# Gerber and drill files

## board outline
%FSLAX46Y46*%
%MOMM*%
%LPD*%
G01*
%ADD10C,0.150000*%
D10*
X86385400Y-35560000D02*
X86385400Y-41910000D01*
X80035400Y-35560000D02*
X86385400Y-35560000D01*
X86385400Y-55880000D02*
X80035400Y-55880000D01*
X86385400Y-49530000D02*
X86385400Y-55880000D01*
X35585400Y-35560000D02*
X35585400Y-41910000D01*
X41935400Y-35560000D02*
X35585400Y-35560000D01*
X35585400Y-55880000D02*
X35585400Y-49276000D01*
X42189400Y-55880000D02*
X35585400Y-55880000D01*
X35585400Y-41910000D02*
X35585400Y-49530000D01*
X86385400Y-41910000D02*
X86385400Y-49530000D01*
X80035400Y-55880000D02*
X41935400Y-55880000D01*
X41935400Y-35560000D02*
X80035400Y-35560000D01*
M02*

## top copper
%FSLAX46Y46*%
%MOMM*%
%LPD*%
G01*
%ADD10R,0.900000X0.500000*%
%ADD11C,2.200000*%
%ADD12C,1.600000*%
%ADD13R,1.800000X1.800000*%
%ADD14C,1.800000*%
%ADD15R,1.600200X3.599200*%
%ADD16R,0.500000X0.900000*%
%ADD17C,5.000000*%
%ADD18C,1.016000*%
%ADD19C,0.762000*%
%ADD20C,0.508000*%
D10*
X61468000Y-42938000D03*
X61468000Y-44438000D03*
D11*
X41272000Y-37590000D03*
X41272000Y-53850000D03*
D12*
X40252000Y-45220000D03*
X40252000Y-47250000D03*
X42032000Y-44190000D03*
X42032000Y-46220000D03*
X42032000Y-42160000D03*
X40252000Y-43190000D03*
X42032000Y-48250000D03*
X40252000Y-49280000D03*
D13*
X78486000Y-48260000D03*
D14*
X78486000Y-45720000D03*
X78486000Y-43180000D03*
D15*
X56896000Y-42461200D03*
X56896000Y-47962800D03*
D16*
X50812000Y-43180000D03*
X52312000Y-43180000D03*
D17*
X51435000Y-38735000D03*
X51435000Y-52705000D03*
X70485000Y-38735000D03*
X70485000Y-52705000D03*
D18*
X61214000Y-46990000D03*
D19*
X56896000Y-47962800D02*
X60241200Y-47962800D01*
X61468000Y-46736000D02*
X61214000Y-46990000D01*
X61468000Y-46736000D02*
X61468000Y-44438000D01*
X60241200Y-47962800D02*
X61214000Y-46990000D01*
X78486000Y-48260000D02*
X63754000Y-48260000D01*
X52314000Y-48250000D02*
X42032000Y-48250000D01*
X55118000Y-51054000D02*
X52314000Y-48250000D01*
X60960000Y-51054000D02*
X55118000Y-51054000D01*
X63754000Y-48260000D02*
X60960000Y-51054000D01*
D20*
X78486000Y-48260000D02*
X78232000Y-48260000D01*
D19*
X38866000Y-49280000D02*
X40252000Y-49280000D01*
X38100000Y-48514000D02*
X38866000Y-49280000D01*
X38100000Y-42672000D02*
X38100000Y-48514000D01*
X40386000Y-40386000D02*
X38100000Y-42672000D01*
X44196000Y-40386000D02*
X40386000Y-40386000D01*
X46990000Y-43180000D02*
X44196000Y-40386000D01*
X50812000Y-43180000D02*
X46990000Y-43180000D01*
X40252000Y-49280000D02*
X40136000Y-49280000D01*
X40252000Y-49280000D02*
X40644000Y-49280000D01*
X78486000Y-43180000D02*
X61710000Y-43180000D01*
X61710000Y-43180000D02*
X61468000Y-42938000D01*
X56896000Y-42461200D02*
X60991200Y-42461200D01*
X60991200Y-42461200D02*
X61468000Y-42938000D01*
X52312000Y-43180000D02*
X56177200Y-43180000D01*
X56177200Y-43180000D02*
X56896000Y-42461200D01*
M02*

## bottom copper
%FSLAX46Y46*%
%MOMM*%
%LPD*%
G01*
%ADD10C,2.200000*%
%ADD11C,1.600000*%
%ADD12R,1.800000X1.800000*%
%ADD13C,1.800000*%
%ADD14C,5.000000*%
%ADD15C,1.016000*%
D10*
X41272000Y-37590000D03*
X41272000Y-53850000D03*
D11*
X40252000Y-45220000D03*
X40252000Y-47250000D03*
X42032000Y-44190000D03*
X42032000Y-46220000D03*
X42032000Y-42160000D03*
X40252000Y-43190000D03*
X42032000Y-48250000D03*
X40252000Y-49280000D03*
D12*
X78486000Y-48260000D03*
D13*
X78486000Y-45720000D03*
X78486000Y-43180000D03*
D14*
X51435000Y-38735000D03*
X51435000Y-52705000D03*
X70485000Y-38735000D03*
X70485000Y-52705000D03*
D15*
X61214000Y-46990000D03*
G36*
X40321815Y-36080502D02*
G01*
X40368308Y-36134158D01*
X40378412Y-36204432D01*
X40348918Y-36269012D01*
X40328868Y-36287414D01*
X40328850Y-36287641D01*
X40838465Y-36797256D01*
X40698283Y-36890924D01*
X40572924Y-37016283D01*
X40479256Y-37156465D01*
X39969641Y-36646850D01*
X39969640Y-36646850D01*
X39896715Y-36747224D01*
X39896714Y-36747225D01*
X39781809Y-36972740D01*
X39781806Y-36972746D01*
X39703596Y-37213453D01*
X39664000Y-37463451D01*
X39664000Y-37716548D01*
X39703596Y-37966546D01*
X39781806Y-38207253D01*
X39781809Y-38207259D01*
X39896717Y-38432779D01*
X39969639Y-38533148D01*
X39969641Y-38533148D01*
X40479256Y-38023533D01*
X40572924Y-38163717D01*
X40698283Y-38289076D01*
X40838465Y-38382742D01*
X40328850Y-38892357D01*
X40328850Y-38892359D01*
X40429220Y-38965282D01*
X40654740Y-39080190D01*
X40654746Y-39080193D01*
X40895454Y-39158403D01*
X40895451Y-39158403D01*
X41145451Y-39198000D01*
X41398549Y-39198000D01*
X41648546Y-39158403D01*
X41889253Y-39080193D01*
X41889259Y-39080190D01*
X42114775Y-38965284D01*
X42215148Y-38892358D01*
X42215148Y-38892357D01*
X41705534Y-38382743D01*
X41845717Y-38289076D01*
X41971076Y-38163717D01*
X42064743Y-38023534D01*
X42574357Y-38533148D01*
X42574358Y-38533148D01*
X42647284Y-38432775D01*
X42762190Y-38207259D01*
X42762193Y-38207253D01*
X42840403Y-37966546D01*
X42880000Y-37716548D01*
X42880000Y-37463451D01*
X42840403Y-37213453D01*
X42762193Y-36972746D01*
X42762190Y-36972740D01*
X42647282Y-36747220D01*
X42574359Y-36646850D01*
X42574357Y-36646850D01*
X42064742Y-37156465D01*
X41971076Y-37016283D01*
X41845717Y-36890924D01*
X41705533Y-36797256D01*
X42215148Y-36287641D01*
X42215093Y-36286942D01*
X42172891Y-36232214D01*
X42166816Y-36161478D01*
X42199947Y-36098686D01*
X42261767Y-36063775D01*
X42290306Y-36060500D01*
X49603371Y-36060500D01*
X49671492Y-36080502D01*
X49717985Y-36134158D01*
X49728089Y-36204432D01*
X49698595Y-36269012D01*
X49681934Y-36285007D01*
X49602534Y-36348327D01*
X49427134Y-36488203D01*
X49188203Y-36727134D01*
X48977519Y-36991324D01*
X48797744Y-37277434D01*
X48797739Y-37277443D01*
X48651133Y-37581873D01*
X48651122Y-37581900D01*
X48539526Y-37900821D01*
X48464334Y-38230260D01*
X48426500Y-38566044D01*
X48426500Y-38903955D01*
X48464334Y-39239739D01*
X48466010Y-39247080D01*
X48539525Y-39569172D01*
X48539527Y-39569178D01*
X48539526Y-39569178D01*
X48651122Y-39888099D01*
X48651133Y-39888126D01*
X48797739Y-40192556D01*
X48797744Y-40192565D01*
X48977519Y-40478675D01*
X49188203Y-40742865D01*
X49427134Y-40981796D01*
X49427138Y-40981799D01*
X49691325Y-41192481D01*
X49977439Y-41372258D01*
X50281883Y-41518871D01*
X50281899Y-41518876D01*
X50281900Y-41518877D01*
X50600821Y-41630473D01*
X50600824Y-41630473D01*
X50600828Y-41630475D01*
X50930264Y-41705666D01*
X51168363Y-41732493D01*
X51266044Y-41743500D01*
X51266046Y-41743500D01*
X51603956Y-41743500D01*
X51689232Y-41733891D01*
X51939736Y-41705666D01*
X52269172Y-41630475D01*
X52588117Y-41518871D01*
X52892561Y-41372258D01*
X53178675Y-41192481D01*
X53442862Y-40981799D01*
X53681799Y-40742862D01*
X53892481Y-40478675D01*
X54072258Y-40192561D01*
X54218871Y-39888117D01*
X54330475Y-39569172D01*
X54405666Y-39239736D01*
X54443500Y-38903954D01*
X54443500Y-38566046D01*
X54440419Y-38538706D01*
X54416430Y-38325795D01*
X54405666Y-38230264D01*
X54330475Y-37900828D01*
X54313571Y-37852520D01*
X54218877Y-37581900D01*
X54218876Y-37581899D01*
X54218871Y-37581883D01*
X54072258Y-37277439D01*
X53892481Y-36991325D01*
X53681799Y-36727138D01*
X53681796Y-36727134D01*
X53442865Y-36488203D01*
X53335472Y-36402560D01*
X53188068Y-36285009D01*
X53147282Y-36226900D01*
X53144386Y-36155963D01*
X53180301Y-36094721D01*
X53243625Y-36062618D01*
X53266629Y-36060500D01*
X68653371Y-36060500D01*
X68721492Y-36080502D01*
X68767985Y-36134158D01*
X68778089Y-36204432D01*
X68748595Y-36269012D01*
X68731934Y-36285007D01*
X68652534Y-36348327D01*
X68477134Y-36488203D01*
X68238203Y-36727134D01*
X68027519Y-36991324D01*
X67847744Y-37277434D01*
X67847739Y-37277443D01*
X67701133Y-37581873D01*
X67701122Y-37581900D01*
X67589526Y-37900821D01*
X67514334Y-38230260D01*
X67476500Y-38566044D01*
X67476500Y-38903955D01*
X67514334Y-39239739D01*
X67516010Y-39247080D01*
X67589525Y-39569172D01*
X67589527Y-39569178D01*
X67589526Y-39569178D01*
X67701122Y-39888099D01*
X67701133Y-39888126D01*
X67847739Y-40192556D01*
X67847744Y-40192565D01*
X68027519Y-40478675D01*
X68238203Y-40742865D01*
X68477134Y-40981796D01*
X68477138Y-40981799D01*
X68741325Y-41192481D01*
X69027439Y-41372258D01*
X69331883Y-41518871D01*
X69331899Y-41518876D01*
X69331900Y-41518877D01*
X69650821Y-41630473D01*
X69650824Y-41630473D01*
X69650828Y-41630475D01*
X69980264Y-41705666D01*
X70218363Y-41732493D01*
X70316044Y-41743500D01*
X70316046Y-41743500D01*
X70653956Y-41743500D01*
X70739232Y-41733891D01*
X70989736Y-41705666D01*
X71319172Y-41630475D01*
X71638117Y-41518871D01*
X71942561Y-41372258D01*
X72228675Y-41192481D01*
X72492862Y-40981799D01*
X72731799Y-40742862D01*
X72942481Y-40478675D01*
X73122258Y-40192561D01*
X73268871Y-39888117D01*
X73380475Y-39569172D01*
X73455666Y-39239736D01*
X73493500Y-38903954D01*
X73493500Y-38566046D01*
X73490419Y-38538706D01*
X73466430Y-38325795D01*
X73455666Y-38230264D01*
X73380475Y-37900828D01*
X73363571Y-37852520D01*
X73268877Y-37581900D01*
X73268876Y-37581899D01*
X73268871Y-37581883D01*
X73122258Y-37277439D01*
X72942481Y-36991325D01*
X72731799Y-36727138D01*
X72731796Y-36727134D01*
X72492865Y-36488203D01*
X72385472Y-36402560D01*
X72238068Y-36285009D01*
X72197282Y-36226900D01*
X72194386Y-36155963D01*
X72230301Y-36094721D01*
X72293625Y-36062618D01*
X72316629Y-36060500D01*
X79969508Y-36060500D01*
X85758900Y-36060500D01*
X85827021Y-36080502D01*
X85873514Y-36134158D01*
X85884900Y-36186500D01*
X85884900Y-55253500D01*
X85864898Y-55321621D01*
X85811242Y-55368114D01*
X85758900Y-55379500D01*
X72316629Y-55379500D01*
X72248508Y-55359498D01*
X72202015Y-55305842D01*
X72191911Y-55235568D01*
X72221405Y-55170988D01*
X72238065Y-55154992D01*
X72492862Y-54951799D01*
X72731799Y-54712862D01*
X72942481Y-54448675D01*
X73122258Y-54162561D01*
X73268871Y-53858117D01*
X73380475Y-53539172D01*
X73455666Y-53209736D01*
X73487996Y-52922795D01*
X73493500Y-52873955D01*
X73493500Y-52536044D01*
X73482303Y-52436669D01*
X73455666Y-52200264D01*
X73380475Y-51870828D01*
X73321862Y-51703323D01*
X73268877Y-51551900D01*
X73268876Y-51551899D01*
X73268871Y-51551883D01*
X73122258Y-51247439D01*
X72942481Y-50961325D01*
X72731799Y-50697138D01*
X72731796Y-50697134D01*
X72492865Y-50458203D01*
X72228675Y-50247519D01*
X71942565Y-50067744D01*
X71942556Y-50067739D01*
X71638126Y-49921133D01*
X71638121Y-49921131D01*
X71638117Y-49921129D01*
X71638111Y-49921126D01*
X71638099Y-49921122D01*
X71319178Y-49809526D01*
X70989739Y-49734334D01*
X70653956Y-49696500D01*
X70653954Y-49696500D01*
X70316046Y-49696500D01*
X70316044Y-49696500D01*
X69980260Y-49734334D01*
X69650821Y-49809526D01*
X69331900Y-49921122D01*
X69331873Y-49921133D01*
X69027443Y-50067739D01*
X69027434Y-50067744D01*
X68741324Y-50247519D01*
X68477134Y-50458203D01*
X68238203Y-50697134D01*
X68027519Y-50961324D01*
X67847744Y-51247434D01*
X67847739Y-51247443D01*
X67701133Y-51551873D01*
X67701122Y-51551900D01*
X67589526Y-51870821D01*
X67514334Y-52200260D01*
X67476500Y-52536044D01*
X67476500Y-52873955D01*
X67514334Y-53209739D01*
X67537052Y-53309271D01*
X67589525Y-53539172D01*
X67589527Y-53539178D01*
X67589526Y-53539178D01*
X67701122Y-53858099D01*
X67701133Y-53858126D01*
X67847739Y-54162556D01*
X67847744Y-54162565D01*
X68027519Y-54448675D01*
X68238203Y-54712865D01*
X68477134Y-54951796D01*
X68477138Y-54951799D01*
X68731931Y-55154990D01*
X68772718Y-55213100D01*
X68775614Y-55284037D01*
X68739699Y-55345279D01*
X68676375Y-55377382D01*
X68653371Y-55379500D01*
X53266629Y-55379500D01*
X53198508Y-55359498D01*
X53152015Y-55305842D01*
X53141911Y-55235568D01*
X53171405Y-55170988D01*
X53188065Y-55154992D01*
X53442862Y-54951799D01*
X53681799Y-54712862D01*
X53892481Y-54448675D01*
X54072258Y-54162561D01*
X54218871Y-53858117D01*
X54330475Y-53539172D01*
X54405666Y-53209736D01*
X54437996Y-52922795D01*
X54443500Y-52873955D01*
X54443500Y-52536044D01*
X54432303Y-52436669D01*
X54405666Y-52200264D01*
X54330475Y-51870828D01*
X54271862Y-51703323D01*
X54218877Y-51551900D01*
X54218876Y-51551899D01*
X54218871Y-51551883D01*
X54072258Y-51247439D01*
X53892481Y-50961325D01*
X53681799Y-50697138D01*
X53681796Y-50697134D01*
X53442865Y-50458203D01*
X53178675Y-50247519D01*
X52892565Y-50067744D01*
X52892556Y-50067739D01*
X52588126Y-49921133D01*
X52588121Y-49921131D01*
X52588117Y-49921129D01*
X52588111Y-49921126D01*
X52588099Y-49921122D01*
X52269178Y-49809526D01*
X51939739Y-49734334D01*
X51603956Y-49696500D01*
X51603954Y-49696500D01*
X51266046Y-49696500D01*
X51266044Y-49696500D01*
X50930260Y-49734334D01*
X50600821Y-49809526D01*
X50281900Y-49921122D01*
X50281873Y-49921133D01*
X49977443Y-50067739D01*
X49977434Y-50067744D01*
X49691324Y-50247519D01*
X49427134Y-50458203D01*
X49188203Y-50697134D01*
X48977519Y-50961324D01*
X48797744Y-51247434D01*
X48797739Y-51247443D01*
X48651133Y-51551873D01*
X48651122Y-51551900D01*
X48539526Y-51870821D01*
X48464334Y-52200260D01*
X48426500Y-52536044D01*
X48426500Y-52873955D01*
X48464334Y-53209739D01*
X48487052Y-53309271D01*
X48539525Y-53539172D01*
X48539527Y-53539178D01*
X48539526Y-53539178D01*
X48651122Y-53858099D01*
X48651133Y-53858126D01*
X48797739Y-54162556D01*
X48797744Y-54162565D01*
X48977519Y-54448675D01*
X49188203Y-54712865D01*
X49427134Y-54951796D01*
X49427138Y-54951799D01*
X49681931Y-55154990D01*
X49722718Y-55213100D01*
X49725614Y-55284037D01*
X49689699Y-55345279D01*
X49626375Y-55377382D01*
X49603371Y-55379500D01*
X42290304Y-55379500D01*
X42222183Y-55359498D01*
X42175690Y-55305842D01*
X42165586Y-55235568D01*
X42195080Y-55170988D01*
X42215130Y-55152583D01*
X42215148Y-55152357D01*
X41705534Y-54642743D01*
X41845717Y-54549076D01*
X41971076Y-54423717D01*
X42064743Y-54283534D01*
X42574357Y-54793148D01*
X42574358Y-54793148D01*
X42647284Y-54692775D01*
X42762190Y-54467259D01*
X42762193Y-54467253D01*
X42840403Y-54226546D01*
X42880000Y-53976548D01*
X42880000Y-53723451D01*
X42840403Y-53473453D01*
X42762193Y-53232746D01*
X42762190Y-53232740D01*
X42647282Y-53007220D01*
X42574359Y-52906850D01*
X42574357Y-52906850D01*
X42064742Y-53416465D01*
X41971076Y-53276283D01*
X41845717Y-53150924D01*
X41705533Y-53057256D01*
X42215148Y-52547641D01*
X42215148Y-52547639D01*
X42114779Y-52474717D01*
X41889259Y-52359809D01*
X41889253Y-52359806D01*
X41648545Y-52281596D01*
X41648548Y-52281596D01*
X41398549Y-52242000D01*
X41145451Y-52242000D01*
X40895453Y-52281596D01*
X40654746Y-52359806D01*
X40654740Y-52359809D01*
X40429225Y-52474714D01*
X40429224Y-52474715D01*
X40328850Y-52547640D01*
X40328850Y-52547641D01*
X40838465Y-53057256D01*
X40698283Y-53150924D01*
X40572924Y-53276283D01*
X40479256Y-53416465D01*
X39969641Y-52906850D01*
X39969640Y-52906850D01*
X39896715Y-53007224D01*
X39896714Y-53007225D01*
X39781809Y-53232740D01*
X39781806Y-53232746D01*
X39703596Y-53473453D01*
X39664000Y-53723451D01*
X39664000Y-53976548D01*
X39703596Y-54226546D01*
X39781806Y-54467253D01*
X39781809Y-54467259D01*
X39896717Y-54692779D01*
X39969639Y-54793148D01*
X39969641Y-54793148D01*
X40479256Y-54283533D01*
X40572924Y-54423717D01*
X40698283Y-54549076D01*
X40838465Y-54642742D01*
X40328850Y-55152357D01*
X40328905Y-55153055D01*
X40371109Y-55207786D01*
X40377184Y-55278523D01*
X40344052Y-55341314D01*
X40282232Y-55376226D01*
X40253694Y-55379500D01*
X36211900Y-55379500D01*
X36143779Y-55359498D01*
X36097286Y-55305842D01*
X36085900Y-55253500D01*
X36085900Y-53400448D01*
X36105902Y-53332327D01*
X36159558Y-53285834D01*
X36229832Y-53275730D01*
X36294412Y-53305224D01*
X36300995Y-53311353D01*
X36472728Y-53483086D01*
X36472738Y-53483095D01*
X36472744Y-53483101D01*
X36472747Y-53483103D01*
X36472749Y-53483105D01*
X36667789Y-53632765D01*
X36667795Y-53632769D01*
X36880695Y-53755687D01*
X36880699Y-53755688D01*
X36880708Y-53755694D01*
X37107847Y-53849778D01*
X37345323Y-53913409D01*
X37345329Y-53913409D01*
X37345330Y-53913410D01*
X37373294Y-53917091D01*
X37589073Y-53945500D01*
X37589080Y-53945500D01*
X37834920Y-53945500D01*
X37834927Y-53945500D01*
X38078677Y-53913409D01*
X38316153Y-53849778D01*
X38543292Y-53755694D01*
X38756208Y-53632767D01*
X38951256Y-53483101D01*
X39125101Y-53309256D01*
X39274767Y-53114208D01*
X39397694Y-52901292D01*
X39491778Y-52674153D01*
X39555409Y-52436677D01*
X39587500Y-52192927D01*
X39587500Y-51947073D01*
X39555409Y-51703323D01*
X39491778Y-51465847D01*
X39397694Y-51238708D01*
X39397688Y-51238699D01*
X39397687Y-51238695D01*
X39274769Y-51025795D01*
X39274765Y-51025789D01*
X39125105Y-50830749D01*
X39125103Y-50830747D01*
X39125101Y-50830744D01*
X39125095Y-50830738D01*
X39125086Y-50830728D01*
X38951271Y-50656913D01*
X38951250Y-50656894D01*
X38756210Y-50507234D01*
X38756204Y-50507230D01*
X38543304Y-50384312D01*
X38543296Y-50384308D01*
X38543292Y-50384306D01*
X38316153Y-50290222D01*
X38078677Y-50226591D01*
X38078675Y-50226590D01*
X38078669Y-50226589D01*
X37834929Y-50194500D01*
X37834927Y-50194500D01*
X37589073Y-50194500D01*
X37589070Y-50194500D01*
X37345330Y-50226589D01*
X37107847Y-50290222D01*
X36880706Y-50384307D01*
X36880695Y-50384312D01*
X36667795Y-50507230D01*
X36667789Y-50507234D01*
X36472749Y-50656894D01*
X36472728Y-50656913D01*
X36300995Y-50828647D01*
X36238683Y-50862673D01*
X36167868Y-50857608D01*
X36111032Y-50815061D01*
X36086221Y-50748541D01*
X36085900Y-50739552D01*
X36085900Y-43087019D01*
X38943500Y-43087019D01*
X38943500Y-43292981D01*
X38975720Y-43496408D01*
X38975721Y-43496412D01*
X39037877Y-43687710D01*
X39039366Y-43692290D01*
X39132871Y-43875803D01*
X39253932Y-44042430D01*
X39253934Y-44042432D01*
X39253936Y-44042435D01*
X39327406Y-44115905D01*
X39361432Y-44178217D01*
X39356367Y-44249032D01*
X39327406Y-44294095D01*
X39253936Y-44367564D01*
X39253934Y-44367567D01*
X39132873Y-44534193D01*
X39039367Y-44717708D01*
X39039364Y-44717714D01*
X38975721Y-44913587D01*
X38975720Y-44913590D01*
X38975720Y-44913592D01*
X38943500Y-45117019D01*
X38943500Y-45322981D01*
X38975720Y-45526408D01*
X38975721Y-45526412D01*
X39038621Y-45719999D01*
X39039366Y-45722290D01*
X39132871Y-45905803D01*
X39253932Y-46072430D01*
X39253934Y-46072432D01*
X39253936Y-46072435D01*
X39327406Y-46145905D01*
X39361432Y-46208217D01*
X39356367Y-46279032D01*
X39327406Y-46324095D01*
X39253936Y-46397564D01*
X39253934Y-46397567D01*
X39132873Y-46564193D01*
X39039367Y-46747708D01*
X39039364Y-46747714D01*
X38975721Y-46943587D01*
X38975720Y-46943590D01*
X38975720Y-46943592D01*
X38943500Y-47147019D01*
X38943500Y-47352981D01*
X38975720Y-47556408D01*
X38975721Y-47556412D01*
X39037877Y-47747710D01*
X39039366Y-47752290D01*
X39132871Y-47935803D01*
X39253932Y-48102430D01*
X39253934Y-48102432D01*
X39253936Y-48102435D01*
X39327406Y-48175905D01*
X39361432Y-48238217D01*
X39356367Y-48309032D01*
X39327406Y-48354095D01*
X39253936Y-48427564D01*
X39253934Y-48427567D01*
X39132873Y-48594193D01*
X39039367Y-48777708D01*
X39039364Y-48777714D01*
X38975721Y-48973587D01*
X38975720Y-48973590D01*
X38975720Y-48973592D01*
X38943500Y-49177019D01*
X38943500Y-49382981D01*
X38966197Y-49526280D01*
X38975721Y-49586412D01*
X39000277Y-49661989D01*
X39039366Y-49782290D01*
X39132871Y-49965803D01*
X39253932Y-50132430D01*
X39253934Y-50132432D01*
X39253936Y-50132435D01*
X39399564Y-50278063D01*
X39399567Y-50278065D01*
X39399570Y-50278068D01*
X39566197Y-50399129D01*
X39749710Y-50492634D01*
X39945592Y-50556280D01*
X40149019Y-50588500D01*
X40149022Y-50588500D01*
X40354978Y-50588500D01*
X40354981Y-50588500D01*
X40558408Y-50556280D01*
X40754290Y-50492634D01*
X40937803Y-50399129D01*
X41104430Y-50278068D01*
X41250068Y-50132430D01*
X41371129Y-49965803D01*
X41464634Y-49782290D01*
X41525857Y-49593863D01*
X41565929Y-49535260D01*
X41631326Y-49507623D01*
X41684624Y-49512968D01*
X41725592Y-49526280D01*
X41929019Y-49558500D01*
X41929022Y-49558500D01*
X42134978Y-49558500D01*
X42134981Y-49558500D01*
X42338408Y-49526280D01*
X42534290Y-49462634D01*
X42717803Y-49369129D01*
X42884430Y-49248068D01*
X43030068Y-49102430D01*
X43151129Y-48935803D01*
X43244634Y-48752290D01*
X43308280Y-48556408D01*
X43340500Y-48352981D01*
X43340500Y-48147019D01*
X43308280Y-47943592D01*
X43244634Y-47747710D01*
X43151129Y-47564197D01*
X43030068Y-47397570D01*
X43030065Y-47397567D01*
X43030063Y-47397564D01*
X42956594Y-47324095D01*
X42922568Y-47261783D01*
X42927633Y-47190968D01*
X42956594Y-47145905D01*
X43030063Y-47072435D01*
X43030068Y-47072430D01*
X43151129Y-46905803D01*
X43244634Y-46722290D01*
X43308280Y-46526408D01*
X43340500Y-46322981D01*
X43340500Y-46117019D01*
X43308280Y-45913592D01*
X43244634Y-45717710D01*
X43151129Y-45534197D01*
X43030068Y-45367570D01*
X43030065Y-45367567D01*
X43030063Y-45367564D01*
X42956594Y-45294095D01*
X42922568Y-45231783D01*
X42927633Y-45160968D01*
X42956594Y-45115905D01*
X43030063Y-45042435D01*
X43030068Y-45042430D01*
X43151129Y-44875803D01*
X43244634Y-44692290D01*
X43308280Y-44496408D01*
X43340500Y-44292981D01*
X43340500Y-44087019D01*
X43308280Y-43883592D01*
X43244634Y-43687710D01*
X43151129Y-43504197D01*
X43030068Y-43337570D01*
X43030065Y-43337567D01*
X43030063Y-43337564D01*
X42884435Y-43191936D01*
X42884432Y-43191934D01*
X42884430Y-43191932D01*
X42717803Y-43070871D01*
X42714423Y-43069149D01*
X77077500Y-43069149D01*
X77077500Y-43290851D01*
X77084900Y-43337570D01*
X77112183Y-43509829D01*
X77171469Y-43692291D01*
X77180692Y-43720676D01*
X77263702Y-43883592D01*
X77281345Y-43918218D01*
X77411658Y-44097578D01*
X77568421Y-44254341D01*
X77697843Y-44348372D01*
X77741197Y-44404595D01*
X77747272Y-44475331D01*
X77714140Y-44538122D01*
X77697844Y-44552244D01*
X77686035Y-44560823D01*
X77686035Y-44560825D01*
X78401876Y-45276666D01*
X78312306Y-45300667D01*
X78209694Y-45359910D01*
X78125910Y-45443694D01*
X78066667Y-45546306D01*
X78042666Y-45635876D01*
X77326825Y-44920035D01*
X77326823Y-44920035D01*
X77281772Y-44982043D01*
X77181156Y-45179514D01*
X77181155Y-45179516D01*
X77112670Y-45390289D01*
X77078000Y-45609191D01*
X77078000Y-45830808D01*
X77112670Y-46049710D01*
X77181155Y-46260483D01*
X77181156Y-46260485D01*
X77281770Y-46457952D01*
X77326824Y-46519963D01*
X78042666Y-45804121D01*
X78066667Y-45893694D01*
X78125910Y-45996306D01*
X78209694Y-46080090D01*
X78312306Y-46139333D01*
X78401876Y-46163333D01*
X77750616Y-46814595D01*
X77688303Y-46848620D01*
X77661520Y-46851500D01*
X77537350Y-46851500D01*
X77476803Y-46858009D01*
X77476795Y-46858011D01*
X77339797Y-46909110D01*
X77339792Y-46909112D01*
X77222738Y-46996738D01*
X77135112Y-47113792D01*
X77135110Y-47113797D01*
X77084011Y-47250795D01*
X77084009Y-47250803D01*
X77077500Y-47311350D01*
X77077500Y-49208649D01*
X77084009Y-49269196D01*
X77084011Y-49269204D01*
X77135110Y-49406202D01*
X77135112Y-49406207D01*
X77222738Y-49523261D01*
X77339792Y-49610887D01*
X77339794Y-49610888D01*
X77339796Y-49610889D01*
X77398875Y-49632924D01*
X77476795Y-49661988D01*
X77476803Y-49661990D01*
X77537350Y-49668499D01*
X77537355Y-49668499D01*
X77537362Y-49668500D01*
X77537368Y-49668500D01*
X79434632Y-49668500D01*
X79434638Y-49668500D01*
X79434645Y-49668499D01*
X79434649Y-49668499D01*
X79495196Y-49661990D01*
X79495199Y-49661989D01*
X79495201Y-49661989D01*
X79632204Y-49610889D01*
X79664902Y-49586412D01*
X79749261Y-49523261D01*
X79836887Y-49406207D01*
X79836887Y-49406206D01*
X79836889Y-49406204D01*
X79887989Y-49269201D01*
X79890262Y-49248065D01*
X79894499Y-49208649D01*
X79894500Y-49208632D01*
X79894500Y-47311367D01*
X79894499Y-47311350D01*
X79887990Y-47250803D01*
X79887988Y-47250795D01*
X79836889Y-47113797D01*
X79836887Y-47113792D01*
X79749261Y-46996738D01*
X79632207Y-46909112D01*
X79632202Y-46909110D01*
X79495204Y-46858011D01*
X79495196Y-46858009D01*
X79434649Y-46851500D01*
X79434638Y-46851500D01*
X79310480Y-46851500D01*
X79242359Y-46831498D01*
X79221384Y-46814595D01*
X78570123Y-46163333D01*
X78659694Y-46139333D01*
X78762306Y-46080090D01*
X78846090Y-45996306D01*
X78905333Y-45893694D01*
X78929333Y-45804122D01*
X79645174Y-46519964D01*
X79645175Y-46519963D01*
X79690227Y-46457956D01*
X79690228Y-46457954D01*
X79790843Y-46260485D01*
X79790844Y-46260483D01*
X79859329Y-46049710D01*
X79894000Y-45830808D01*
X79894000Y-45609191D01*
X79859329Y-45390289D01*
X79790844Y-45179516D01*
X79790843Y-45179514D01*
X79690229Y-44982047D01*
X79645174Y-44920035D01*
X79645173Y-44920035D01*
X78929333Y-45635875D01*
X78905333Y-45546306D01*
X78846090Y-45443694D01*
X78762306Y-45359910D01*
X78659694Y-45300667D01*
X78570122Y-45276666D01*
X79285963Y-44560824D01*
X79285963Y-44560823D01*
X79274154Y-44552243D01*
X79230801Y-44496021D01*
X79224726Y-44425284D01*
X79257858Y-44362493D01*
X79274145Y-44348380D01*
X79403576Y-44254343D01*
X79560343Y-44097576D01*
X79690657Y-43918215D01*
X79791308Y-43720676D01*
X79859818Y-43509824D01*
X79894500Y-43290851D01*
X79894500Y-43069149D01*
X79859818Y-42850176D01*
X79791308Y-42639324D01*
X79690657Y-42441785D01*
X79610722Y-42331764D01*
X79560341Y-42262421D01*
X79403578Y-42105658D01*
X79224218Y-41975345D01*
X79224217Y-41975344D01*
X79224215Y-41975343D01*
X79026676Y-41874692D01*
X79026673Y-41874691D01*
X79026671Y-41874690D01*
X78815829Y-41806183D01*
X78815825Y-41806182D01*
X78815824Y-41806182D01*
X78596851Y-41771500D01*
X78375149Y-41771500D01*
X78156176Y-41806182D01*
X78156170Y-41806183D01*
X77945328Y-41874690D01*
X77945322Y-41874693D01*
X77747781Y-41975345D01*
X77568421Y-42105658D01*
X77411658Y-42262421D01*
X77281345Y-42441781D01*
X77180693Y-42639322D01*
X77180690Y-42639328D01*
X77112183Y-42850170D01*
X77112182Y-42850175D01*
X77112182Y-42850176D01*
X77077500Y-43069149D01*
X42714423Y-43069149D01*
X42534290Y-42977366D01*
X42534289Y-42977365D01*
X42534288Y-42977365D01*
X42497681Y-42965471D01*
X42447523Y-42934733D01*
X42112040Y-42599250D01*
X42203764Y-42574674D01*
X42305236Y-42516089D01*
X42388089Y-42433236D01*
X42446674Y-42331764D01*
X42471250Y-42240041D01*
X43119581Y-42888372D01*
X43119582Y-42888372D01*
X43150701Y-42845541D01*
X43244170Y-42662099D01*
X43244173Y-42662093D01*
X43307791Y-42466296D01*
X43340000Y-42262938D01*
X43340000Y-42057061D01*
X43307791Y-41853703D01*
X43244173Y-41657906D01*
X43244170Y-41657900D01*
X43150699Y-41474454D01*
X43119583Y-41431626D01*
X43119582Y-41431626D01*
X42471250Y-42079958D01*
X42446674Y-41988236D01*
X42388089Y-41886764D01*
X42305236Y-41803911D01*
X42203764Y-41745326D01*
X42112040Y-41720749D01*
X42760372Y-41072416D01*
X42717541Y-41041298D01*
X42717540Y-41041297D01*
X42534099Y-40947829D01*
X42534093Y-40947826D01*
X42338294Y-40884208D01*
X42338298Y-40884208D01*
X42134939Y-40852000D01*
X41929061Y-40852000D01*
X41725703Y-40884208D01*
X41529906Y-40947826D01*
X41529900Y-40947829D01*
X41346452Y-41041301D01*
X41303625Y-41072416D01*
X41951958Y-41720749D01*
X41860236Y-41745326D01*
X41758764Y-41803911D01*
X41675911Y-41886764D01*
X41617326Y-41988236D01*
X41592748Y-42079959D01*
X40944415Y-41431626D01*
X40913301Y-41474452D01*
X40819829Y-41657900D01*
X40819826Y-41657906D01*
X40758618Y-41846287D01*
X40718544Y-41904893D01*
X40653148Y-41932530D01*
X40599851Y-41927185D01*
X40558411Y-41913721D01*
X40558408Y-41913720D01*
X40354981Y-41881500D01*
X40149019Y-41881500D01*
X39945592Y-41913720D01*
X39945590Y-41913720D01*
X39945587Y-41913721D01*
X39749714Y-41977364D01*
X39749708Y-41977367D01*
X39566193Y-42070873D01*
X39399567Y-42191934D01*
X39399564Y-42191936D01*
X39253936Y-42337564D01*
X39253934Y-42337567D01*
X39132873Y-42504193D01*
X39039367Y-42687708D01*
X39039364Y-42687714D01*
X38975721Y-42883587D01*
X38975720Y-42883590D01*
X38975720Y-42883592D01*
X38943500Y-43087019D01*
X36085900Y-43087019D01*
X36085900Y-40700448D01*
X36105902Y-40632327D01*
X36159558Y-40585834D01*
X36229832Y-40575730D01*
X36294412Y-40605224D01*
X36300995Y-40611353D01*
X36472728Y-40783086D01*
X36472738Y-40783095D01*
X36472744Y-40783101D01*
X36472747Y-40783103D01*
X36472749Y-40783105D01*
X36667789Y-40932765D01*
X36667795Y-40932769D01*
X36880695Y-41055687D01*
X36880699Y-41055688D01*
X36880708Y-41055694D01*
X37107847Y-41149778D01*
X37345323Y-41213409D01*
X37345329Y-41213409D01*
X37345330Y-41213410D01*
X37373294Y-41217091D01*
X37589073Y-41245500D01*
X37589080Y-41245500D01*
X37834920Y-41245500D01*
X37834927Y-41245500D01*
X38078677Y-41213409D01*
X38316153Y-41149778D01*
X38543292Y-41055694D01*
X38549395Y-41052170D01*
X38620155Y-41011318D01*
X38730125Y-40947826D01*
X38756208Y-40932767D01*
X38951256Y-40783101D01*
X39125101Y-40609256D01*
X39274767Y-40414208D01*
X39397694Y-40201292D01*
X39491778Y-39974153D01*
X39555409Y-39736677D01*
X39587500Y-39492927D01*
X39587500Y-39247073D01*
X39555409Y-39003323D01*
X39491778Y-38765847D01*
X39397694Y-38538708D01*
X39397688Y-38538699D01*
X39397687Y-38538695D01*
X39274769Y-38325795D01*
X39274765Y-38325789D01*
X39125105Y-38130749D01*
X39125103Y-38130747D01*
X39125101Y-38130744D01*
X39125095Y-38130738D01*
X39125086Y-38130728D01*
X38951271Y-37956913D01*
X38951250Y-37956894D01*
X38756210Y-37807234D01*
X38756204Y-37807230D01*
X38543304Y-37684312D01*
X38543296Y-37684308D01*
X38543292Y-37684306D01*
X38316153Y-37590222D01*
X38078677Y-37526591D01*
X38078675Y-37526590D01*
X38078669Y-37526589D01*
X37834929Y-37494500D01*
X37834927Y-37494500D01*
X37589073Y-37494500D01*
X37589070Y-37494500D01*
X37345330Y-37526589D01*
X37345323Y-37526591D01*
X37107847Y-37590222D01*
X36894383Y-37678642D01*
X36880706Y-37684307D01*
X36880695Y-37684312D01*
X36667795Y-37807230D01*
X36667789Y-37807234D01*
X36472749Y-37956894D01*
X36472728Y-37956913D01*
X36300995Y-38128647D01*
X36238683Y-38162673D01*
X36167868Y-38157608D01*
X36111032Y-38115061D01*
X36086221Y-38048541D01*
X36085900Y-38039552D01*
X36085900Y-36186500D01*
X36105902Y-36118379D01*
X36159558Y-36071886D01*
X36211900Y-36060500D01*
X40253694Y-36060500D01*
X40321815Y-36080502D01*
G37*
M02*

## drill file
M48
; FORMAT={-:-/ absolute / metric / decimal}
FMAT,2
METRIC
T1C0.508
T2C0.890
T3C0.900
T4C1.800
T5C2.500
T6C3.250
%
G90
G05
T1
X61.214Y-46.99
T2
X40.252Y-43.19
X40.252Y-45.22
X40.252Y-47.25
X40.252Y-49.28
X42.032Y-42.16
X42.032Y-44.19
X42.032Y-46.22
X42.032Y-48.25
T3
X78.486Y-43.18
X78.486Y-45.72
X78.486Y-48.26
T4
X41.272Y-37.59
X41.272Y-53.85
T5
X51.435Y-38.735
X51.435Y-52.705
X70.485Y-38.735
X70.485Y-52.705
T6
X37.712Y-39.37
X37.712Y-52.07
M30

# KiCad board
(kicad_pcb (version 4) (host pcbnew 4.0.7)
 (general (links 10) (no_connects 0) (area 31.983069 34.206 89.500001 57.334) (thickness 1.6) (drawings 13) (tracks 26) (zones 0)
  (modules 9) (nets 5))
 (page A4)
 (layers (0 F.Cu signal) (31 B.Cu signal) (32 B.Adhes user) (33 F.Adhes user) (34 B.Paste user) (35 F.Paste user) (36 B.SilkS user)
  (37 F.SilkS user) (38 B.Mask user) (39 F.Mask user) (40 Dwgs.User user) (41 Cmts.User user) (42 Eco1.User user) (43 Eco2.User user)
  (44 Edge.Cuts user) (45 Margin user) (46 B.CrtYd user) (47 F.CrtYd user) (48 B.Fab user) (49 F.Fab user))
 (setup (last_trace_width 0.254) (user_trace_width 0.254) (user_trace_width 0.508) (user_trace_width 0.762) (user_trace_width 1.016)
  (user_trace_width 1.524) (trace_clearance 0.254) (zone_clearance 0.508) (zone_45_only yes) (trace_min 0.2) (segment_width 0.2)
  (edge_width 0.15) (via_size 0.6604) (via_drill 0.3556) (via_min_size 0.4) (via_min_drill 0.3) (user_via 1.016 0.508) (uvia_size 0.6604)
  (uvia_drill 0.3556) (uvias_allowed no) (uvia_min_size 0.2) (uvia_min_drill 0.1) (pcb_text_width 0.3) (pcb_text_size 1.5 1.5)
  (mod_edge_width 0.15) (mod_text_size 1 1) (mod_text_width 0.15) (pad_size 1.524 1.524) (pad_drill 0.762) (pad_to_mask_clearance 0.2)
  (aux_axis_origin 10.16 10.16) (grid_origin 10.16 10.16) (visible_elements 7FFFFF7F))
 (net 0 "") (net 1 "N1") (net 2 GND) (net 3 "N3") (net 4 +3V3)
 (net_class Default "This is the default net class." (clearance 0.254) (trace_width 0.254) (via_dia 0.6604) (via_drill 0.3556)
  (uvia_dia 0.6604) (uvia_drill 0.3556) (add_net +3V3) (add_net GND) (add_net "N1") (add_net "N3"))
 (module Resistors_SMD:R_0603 (layer F.Cu) (at 61.468 43.688 270)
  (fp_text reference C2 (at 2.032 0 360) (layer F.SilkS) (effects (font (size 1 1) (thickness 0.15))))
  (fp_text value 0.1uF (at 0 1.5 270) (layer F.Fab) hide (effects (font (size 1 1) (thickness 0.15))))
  (pad 1 smd rect (at -0.75 0 270) (size 0.5 0.9) (layers F.Cu F.Paste F.Mask) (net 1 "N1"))
  (pad 2 smd rect (at 0.75 0 270) (size 0.5 0.9) (layers F.Cu F.Paste F.Mask) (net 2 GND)))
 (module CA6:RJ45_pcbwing (layer F.Cu) (at 40.132 45.72 270)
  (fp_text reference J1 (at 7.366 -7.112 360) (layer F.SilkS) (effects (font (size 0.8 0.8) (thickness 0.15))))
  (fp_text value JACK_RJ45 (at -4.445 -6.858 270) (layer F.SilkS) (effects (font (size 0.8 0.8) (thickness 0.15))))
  (pad 8 thru_hole circle (at -8.13 -1.14 270) (size 2.2 2.2) (drill 1.8) (layers *.Cu *.Mask F.SilkS) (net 2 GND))
  (pad 8 thru_hole circle (at 8.13 -1.14 270) (size 2.2 2.2) (drill 1.8) (layers *.Cu *.Mask F.SilkS) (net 2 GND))
  (pad "" np_thru_hole circle (at -6.35 2.42 270) (size 3.25 3.25) (drill 3.25) (layers *.Cu *.Mask F.SilkS))
  (pad "" np_thru_hole circle (at 6.35 2.42 270) (size 3.25 3.25) (drill 3.25) (layers *.Cu *.Mask F.SilkS))
  (pad 5 thru_hole circle (at -0.5 -0.12 270) (size 1.6 1.6) (drill 0.89) (layers *.Cu *.Mask F.SilkS))
  (pad 3 thru_hole circle (at 1.53 -0.12 270) (size 1.6 1.6) (drill 0.89) (layers *.Cu *.Mask F.SilkS))
  (pad 6 thru_hole circle (at -1.53 -1.9 270) (size 1.6 1.6) (drill 0.89) (layers *.Cu *.Mask F.SilkS))
  (pad 4 thru_hole circle (at 0.5 -1.9 270) (size 1.6 1.6) (drill 0.89) (layers *.Cu *.Mask F.SilkS))
  (pad 8 thru_hole circle (at -3.56 -1.9 270) (size 1.6 1.6) (drill 0.89) (layers *.Cu *.Mask F.SilkS) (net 2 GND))
  (pad 7 thru_hole circle (at -2.53 -0.12 270) (size 1.6 1.6) (drill 0.89) (layers *.Cu *.Mask F.SilkS))
  (pad 2 thru_hole circle (at 2.53 -1.9 270) (size 1.6 1.6) (drill 0.89) (layers *.Cu *.Mask F.SilkS) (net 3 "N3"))
  (pad 1 thru_hole circle (at 3.56 -0.12 270) (size 1.6 1.6) (drill 0.89) (layers *.Cu *.Mask F.SilkS) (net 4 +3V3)))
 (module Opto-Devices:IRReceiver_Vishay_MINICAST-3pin (layer F.Cu) (at 78.486 48.26 90)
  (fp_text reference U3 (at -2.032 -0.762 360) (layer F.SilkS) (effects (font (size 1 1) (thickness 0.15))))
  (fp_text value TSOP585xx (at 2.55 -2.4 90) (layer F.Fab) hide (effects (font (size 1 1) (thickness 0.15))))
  (pad 1 thru_hole rect (at 0 0 90) (size 1.8 1.8) (drill 0.9) (layers *.Cu *.Mask) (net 3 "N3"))
  (pad 2 thru_hole circle (at 2.54 0 90) (size 1.8 1.8) (drill 0.9) (layers *.Cu *.Mask) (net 2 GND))
  (pad 3 thru_hole circle (at 5.08 0 90) (size 1.8 1.8) (drill 0.9) (layers *.Cu *.Mask) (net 1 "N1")))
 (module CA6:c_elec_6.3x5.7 (layer F.Cu) (at 56.896 45.212 90)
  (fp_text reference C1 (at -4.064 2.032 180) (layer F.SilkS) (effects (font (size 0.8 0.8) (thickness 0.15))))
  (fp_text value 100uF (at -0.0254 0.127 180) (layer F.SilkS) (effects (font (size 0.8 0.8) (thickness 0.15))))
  (pad 1 smd rect (at 2.7508 0 90) (size 3.5992 1.6002) (layers F.Cu F.Paste F.Mask) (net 1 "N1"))
  (pad 2 smd rect (at -2.7508 0 90) (size 3.5992 1.6002) (layers F.Cu F.Paste F.Mask) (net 2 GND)))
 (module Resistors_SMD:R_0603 (layer F.Cu) (at 51.562 43.18)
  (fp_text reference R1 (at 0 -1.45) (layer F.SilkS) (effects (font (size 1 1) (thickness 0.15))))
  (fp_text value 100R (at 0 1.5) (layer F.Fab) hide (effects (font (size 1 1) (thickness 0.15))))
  (pad 1 smd rect (at -0.75 0) (size 0.5 0.9) (layers F.Cu F.Paste F.Mask) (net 4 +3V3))
  (pad 2 smd rect (at 0.75 0) (size 0.5 0.9) (layers F.Cu F.Paste F.Mask) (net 1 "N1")))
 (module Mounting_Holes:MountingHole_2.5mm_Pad (layer F.Cu) (at 51.435 38.735)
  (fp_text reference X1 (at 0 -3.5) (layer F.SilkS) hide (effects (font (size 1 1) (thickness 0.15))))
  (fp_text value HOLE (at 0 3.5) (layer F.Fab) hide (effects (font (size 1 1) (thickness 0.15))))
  (pad 1 thru_hole circle (at 0 0) (size 5 5) (drill 2.5) (layers *.Cu *.Mask)))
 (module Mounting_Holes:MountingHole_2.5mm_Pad (layer F.Cu) (at 51.435 52.705)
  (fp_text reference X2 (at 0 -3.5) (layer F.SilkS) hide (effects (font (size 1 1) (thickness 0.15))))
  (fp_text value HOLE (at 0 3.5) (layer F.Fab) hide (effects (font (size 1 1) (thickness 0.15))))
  (pad 1 thru_hole circle (at 0 0) (size 5 5) (drill 2.5) (layers *.Cu *.Mask)))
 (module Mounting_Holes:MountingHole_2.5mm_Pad (layer F.Cu) (at 70.485 38.735)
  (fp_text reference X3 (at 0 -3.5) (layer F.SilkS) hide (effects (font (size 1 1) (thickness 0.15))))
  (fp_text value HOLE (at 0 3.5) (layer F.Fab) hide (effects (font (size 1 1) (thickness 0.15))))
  (pad 1 thru_hole circle (at 0 0) (size 5 5) (drill 2.5) (layers *.Cu *.Mask)))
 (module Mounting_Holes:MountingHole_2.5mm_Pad (layer F.Cu) (at 70.485 52.705)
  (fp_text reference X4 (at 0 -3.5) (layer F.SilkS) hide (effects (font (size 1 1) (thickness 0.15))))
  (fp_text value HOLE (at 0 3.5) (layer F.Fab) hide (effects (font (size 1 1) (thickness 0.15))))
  (pad 1 thru_hole circle (at 0 0) (size 5 5) (drill 2.5) (layers *.Cu *.Mask)))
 (gr_line (start 86.3854 35.56) (end 86.3854 41.91) (angle 90) (layer Edge.Cuts) (width 0.15))
 (gr_line (start 80.0354 35.56) (end 86.3854 35.56) (angle 90) (layer Edge.Cuts) (width 0.15))
 (gr_line (start 86.3854 55.88) (end 80.0354 55.88) (angle 90) (layer Edge.Cuts) (width 0.15))
 (gr_line (start 86.3854 49.53) (end 86.3854 55.88) (angle 90) (layer Edge.Cuts) (width 0.15))
 (gr_line (start 35.5854 35.56) (end 35.5854 41.91) (angle 90) (layer Edge.Cuts) (width 0.15))
 (gr_line (start 41.9354 35.56) (end 35.5854 35.56) (angle 90) (layer Edge.Cuts) (width 0.15))
 (gr_line (start 35.5854 55.88) (end 35.5854 49.276) (angle 90) (layer Edge.Cuts) (width 0.15))
 (gr_line (start 42.1894 55.88) (end 35.5854 55.88) (angle 90) (layer Edge.Cuts) (width 0.15))
 (gr_line (start 35.5854 41.91) (end 35.5854 49.53) (angle 90) (layer Edge.Cuts) (width 0.15))
 (gr_line (start 86.3854 41.91) (end 86.3854 49.53) (angle 90) (layer Edge.Cuts) (width 0.15))
 (gr_line (start 80.0354 55.88) (end 41.9354 55.88) (angle 90) (layer Edge.Cuts) (width 0.15))
 (gr_line (start 41.9354 35.56) (end 80.0354 35.56) (angle 90) (layer Edge.Cuts) (width 0.15))
 (segment (start 56.896 47.9628) (end 60.2412 47.9628) (width 0.762) (layer F.Cu) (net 2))
 (segment (start 61.468 46.736) (end 61.214 46.99) (width 0.762) (layer F.Cu) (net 2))
 (via (at 61.214 46.99) (size 1.016) (drill 0.508) (layers F.Cu B.Cu) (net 2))
 (segment (start 61.468 46.736) (end 61.468 44.438) (width 0.762) (layer F.Cu) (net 2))
 (segment (start 60.2412 47.9628) (end 61.214 46.99) (width 0.762) (layer F.Cu) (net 2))
 (segment (start 78.486 48.26) (end 63.754 48.26) (width 0.762) (layer F.Cu) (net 3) (status 10))
 (segment (start 52.314 48.25) (end 42.032 48.25) (width 0.762) (layer F.Cu) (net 3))
 (segment (start 55.118 51.054) (end 52.314 48.25) (width 0.762) (layer F.Cu) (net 3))
 (segment (start 60.96 51.054) (end 55.118 51.054) (width 0.762) (layer F.Cu) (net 3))
 (segment (start 63.754 48.26) (end 60.96 51.054) (width 0.762) (layer F.Cu) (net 3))
 (segment (start 78.486 48.26) (end 78.232 48.26) (width 0.508) (layer F.Cu) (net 3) (status 30))
 (segment (start 38.866 49.28) (end 40.252 49.28) (width 0.762) (layer F.Cu) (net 4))
 (segment (start 38.1 48.514) (end 38.866 49.28) (width 0.762) (layer F.Cu) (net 4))
 (segment (start 38.1 42.672) (end 38.1 48.514) (width 0.762) (layer F.Cu) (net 4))
 (segment (start 40.386 40.386) (end 38.1 42.672) (width 0.762) (layer F.Cu) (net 4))
 (segment (start 44.196 40.386) (end 40.386 40.386) (width 0.762) (layer F.Cu) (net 4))
 (segment (start 46.99 43.18) (end 44.196 40.386) (width 0.762) (layer F.Cu) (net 4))
 (segment (start 50.812 43.18) (end 46.99 43.18) (width 0.762) (layer F.Cu) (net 4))
 (segment (start 40.252 49.28) (end 40.136 49.28) (width 0.762) (layer F.Cu) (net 4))
 (segment (start 40.252 49.28) (end 40.644 49.28) (width 0.762) (layer F.Cu) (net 4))
 (segment (start 78.486 43.18) (end 61.71 43.18) (width 0.762) (layer F.Cu) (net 1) (status 10))
 (segment (start 61.71 43.18) (end 61.468 42.938) (width 0.762) (layer F.Cu) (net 1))
 (segment (start 56.896 42.4612) (end 60.9912 42.4612) (width 0.762) (layer F.Cu) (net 1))
 (segment (start 60.9912 42.4612) (end 61.468 42.938) (width 0.762) (layer F.Cu) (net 1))
 (segment (start 52.312 43.18) (end 56.1772 43.18) (width 0.762) (layer F.Cu) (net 1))
 (segment (start 56.1772 43.18) (end 56.896 42.4612) (width 0.762) (layer F.Cu) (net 1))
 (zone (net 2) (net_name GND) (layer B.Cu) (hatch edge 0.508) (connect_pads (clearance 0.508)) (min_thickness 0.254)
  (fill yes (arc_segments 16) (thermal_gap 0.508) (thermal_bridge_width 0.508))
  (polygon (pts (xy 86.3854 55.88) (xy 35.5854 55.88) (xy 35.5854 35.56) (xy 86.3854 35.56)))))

